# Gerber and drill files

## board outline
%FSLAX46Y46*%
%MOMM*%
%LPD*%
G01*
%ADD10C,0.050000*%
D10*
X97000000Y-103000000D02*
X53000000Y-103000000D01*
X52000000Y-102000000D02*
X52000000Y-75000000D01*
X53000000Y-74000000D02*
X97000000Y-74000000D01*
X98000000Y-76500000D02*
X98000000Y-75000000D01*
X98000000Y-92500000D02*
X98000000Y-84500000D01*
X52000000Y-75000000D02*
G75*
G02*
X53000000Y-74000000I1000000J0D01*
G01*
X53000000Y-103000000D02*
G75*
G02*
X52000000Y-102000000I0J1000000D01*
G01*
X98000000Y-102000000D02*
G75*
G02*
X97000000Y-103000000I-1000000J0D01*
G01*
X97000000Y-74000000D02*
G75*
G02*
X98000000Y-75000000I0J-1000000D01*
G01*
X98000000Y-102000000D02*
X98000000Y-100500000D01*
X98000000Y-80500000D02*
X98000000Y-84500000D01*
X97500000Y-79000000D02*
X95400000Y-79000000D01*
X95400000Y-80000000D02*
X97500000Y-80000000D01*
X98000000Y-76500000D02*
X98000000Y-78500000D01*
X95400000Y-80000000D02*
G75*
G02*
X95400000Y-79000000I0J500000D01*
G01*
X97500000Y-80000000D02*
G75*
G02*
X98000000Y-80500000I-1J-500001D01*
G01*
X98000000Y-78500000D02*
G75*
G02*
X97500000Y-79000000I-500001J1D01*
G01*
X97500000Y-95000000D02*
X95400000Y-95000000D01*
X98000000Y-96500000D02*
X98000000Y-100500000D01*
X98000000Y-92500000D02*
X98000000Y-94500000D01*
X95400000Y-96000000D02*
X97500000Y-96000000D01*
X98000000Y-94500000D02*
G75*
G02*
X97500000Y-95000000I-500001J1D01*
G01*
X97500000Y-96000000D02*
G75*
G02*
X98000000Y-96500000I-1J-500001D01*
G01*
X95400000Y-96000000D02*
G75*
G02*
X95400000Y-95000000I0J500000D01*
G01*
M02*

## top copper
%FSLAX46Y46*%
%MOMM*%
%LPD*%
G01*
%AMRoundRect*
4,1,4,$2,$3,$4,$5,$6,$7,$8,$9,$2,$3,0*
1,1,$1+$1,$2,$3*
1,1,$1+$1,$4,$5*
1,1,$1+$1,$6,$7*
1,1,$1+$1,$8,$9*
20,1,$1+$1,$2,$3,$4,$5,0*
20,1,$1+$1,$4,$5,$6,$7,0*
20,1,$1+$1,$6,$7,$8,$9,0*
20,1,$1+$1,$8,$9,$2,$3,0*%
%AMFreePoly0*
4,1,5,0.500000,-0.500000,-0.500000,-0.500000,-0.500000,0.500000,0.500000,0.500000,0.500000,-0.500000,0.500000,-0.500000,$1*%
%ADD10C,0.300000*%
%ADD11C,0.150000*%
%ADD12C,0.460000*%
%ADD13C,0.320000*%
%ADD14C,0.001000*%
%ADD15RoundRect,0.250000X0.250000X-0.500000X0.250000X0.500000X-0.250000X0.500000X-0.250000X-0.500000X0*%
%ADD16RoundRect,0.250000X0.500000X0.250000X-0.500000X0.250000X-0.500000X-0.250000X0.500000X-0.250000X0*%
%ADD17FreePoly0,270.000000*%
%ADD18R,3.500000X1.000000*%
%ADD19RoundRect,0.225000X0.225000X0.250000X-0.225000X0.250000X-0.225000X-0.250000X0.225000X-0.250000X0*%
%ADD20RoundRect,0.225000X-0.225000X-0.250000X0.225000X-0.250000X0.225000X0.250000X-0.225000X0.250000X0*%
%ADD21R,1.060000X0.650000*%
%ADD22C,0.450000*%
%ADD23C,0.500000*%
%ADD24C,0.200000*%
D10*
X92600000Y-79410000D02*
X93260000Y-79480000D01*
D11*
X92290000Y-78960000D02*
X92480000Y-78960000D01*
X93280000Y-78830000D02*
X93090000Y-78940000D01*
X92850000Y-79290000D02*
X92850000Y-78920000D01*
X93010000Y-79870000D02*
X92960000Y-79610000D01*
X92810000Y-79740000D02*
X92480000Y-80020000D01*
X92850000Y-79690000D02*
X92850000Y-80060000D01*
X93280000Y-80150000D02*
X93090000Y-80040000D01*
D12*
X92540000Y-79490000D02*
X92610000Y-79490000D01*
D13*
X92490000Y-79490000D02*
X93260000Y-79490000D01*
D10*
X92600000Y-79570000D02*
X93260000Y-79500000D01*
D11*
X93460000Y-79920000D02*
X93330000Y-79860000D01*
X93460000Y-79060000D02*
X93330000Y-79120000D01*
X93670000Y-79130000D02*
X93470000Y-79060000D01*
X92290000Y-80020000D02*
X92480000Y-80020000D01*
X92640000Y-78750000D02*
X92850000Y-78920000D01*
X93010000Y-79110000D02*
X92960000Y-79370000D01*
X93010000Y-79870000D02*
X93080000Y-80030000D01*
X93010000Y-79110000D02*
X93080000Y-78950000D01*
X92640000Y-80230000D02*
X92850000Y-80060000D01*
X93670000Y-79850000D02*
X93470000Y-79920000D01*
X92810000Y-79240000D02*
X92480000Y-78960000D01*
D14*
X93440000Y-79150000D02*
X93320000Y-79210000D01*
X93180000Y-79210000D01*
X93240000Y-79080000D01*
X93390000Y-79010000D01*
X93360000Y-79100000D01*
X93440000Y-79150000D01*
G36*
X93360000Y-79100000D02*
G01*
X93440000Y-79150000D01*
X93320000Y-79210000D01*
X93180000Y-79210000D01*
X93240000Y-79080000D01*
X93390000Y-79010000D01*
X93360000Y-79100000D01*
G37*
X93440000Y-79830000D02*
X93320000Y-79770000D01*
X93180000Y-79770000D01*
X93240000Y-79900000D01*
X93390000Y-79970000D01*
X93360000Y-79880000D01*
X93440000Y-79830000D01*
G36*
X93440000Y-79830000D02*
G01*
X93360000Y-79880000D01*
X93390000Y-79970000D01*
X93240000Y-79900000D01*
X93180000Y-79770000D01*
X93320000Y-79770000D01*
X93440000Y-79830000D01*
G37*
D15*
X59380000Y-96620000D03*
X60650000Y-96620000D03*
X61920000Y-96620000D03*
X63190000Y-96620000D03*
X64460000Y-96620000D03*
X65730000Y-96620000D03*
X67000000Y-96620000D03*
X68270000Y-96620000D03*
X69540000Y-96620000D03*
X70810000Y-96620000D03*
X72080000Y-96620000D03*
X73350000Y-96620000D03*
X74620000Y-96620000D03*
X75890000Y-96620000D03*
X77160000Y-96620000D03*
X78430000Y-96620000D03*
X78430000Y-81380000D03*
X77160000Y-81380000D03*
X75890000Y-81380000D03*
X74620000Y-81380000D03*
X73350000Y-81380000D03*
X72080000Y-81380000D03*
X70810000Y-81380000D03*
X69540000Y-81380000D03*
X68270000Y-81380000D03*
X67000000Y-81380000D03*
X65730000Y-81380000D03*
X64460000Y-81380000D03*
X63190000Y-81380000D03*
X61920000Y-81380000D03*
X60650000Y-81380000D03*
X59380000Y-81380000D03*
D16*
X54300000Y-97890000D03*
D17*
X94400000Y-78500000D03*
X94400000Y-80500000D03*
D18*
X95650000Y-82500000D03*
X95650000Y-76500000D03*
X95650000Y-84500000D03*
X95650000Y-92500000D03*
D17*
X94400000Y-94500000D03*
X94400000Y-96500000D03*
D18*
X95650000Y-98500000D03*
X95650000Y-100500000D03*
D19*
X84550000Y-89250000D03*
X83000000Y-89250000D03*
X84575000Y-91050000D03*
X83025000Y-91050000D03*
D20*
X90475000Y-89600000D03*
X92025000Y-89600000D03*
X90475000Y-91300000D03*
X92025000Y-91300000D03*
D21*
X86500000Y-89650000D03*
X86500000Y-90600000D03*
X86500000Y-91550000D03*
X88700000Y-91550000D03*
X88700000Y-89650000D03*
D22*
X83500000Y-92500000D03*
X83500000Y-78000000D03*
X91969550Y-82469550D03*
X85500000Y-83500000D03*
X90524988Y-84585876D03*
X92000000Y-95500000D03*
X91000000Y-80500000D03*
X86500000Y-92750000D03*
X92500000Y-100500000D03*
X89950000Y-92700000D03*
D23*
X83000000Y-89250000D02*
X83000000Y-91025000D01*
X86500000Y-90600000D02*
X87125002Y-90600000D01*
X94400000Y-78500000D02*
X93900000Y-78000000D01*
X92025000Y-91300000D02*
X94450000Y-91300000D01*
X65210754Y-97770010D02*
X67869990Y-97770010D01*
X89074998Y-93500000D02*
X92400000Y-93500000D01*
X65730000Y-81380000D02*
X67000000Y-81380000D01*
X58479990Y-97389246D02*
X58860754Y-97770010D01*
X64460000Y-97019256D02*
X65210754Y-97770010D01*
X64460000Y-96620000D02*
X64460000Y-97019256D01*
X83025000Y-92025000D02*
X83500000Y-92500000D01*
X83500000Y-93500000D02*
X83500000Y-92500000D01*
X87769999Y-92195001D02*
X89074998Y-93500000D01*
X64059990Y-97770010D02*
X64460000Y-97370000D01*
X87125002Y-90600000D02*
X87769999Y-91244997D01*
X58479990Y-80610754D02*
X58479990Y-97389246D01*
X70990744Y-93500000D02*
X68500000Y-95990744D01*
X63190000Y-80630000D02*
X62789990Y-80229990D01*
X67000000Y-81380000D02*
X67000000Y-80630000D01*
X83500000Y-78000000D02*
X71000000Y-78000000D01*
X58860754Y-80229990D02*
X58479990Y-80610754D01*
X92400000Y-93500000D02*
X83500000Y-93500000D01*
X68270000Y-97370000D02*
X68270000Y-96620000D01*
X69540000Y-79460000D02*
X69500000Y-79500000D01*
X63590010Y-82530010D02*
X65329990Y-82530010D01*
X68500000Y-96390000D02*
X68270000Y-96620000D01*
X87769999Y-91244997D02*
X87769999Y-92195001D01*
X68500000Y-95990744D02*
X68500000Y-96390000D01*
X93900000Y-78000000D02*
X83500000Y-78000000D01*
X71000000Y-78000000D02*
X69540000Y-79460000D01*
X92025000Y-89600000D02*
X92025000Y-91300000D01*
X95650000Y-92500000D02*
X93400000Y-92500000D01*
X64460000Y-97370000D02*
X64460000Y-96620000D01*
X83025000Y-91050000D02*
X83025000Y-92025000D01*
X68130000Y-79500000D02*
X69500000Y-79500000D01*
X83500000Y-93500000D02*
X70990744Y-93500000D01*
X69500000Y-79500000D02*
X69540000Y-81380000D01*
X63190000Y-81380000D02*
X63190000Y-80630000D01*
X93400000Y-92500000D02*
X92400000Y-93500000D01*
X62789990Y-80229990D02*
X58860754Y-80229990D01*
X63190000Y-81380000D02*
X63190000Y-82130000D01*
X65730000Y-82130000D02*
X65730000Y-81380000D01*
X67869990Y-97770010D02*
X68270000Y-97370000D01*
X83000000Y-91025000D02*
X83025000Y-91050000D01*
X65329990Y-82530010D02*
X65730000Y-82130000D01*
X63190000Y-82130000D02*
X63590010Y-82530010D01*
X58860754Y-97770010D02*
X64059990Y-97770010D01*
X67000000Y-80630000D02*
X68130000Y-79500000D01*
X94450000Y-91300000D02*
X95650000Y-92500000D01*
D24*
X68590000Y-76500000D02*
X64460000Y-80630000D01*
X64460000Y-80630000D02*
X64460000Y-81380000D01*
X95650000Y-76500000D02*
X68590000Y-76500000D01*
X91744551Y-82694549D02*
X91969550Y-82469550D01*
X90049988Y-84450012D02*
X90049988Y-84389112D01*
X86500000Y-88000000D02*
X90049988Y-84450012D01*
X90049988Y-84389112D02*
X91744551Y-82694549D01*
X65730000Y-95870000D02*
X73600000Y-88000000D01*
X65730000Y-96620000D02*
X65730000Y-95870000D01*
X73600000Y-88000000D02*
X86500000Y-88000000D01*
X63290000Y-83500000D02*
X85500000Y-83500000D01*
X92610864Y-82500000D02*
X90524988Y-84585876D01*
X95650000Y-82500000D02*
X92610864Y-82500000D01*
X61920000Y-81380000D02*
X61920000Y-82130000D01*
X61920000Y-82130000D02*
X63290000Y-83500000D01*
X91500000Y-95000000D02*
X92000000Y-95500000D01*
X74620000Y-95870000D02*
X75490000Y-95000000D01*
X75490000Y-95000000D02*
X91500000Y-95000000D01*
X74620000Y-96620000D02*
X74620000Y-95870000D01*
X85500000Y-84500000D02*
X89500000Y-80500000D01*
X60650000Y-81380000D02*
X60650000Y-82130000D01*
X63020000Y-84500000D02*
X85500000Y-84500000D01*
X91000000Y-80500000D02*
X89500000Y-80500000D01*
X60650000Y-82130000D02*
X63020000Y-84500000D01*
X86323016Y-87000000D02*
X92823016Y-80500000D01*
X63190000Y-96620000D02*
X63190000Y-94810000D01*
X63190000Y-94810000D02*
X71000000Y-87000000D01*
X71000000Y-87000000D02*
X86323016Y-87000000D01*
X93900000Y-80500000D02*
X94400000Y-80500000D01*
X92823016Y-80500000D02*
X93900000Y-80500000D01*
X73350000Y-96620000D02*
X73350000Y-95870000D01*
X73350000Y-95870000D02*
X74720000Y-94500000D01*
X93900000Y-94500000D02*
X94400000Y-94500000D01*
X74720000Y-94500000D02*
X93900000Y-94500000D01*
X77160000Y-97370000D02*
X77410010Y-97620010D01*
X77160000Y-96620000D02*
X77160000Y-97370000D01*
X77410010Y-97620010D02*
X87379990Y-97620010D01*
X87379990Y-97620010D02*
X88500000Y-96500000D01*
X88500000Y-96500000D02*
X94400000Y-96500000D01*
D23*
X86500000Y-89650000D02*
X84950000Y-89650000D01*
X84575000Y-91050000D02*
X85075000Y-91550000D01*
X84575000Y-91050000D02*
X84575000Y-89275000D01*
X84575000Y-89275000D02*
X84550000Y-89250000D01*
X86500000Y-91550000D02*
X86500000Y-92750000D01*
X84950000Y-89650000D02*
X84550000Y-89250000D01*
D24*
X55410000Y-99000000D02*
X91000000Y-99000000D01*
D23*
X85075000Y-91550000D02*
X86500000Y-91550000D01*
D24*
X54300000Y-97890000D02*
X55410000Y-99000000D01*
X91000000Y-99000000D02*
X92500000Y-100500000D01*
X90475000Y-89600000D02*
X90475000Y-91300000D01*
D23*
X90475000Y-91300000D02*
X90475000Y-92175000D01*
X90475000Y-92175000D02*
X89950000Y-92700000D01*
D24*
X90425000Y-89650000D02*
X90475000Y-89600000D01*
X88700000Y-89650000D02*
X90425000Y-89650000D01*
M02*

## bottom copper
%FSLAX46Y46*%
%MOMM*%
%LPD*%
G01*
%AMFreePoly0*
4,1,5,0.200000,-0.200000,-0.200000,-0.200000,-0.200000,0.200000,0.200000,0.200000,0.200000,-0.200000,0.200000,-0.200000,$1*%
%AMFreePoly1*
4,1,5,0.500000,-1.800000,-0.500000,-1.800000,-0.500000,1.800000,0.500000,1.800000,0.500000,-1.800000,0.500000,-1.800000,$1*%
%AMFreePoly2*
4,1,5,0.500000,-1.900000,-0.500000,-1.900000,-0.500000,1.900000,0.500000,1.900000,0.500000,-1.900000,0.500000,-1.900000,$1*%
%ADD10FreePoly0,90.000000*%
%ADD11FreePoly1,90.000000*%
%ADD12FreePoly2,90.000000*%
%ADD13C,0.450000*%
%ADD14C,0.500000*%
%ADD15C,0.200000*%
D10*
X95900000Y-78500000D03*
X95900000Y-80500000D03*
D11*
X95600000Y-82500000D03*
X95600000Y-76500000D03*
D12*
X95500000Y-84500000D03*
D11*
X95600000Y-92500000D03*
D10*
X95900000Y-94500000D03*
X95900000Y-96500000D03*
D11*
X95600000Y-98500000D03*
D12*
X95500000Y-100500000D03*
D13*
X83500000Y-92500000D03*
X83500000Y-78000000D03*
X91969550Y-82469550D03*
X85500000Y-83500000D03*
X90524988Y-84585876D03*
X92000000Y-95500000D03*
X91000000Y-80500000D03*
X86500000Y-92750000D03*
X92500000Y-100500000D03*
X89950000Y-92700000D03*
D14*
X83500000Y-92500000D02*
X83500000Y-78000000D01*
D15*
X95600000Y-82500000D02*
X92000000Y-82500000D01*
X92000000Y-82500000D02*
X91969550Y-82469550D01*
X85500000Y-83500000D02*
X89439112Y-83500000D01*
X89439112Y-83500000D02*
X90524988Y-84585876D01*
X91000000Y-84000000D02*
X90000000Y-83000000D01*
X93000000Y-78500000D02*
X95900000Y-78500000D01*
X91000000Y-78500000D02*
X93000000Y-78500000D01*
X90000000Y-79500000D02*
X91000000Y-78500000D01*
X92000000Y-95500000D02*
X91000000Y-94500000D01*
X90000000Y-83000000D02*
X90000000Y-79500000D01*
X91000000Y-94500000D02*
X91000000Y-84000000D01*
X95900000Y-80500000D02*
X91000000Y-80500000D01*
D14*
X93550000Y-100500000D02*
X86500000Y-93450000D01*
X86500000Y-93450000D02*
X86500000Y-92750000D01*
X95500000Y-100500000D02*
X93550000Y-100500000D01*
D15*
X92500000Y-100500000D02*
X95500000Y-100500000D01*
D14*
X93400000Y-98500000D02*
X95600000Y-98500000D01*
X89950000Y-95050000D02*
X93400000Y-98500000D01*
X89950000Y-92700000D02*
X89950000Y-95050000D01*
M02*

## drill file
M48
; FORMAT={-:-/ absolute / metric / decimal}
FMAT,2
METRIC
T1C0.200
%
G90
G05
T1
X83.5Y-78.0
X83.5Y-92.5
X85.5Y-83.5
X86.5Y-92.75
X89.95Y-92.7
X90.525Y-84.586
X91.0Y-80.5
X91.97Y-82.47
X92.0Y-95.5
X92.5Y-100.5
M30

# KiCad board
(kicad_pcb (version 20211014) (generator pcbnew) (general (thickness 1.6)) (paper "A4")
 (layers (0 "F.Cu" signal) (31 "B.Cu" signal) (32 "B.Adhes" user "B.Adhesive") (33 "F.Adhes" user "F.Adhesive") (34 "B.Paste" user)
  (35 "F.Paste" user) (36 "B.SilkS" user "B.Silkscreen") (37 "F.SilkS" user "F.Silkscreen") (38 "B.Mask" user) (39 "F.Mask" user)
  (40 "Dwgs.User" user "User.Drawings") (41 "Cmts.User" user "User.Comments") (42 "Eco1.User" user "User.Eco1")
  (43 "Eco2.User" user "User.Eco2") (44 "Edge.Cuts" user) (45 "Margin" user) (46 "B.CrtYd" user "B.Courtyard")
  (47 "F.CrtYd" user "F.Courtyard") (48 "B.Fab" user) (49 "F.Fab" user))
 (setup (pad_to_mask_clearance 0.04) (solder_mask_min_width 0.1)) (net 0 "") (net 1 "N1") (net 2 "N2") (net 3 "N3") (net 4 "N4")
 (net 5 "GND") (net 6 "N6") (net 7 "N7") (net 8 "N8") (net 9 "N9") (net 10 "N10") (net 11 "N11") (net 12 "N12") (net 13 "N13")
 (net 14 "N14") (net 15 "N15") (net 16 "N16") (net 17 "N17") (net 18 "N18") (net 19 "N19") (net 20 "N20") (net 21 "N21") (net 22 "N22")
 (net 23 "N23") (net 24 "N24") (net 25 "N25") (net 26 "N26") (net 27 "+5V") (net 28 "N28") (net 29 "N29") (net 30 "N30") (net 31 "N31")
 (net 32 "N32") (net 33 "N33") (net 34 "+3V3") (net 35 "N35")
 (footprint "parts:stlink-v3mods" (layer "F.Cu") (at 67 89 90)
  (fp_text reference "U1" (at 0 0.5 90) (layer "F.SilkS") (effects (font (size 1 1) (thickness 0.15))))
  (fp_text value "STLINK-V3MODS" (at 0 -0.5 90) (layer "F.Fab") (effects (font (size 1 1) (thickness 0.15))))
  (pad "1" smd roundrect locked (at -7.62 -7.62 90) (size 1.5 1) (layers "F.Cu" "F.Paste" "F.Mask") (roundrect_rratio 0.25) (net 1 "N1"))
  (pad "2" smd roundrect locked (at -7.62 -6.35 90) (size 1.5 1) (layers "F.Cu" "F.Paste" "F.Mask") (roundrect_rratio 0.25) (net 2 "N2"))
  (pad "3" smd roundrect locked (at -7.62 -5.08 90) (size 1.5 1) (layers "F.Cu" "F.Paste" "F.Mask") (roundrect_rratio 0.25) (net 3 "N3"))
  (pad "4" smd roundrect locked (at -7.62 -3.81 90) (size 1.5 1) (layers "F.Cu" "F.Paste" "F.Mask") (roundrect_rratio 0.25) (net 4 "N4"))
  (pad "5" smd roundrect locked (at -7.62 -2.54 90) (size 1.5 1) (layers "F.Cu" "F.Paste" "F.Mask") (roundrect_rratio 0.25) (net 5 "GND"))
  (pad "6" smd roundrect locked (at -7.62 -1.27 90) (size 1.5 1) (layers "F.Cu" "F.Paste" "F.Mask") (roundrect_rratio 0.25) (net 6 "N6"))
  (pad "7" smd roundrect locked (at -7.62 0 90) (size 1.5 1) (layers "F.Cu" "F.Paste" "F.Mask") (roundrect_rratio 0.25) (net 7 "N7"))
  (pad "8" smd roundrect locked (at -7.62 1.27 90) (size 1.5 1) (layers "F.Cu" "F.Paste" "F.Mask") (roundrect_rratio 0.25) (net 5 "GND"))
  (pad "9" smd roundrect locked (at -7.62 2.54 90) (size 1.5 1) (layers "F.Cu" "F.Paste" "F.Mask") (roundrect_rratio 0.25) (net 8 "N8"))
  (pad "10" smd roundrect locked (at -7.62 3.81 90) (size 1.5 1) (layers "F.Cu" "F.Paste" "F.Mask") (roundrect_rratio 0.25) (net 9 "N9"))
  (pad "11" smd roundrect locked (at -7.62 5.08 90) (size 1.5 1) (layers "F.Cu" "F.Paste" "F.Mask") (roundrect_rratio 0.25) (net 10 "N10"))
  (pad "12" smd roundrect locked (at -7.62 6.35 90) (size 1.5 1) (layers "F.Cu" "F.Paste" "F.Mask") (roundrect_rratio 0.25) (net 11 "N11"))
  (pad "13" smd roundrect locked (at -7.62 7.62 90) (size 1.5 1) (layers "F.Cu" "F.Paste" "F.Mask") (roundrect_rratio 0.25) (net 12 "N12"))
  (pad "14" smd roundrect locked (at -7.62 8.89 90) (size 1.5 1) (layers "F.Cu" "F.Paste" "F.Mask") (roundrect_rratio 0.25) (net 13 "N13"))
  (pad "15" smd roundrect locked (at -7.62 10.16 90) (size 1.5 1) (layers "F.Cu" "F.Paste" "F.Mask") (roundrect_rratio 0.25) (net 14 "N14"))
  (pad "16" smd roundrect locked (at -7.62 11.43 90) (size 1.5 1) (layers "F.Cu" "F.Paste" "F.Mask") (roundrect_rratio 0.25) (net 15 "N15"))
  (pad "17" smd roundrect locked (at 7.62 11.43 90) (size 1.5 1) (layers "F.Cu" "F.Paste" "F.Mask") (roundrect_rratio 0.25) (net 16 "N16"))
  (pad "18" smd roundrect locked (at 7.62 10.16 90) (size 1.5 1) (layers "F.Cu" "F.Paste" "F.Mask") (roundrect_rratio 0.25) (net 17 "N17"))
  (pad "19" smd roundrect locked (at 7.62 8.89 90) (size 1.5 1) (layers "F.Cu" "F.Paste" "F.Mask") (roundrect_rratio 0.25) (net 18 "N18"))
  (pad "20" smd roundrect locked (at 7.62 7.62 90) (size 1.5 1) (layers "F.Cu" "F.Paste" "F.Mask") (roundrect_rratio 0.25) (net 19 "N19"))
  (pad "21" smd roundrect locked (at 7.62 6.35 90) (size 1.5 1) (layers "F.Cu" "F.Paste" "F.Mask") (roundrect_rratio 0.25) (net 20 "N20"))
  (pad "22" smd roundrect locked (at 7.62 5.08 90) (size 1.5 1) (layers "F.Cu" "F.Paste" "F.Mask") (roundrect_rratio 0.25))
  (pad "23" smd roundrect locked (at 7.62 3.81 90) (size 1.5 1) (layers "F.Cu" "F.Paste" "F.Mask") (roundrect_rratio 0.25) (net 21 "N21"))
  (pad "24" smd roundrect locked (at 7.62 2.54 90) (size 1.5 1) (layers "F.Cu" "F.Paste" "F.Mask") (roundrect_rratio 0.25) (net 5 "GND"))
  (pad "25" smd roundrect locked (at 7.62 1.27 90) (size 1.5 1) (layers "F.Cu" "F.Paste" "F.Mask") (roundrect_rratio 0.25) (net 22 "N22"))
  (pad "26" smd roundrect locked (at 7.62 0 90) (size 1.5 1) (layers "F.Cu" "F.Paste" "F.Mask") (roundrect_rratio 0.25) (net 5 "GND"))
  (pad "27" smd roundrect locked (at 7.62 -1.27 90) (size 1.5 1) (layers "F.Cu" "F.Paste" "F.Mask") (roundrect_rratio 0.25) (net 5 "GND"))
  (pad "28" smd roundrect locked (at 7.62 -2.54 90) (size 1.5 1) (layers "F.Cu" "F.Paste" "F.Mask") (roundrect_rratio 0.25) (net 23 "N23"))
  (pad "29" smd roundrect locked (at 7.62 -3.81 90) (size 1.5 1) (layers "F.Cu" "F.Paste" "F.Mask") (roundrect_rratio 0.25) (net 5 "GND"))
  (pad "30" smd roundrect locked (at 7.62 -5.08 90) (size 1.5 1) (layers "F.Cu" "F.Paste" "F.Mask") (roundrect_rratio 0.25) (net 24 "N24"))
  (pad "31" smd roundrect locked (at 7.62 -6.35 90) (size 1.5 1) (layers "F.Cu" "F.Paste" "F.Mask") (roundrect_rratio 0.25) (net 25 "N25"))
  (pad "32" smd roundrect locked (at 7.62 -7.62 90) (size 1.5 1) (layers "F.Cu" "F.Paste" "F.Mask") (roundrect_rratio 0.25) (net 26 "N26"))
  (pad "33" smd roundrect locked (at -8.89 -12.7 180) (size 1.5 1) (layers "F.Cu" "F.Paste" "F.Mask") (roundrect_rratio 0.25) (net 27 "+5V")))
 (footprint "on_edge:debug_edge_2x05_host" (layer "F.Cu") (at 98 80.5 -90)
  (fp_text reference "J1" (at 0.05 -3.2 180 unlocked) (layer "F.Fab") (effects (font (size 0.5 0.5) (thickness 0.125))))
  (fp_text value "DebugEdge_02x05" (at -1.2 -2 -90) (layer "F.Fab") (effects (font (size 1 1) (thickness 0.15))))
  (fp_line (start -1.09 5.4) (end -1.02 4.74) (layer "F.Cu") (width 0.3))
  (fp_line (start -1.54 5.71) (end -1.54 5.52) (layer "F.Cu") (width 0.15))
  (fp_line (start -1.67 4.72) (end -1.56 4.91) (layer "F.Cu") (width 0.15))
  (fp_line (start -1.21 5.15) (end -1.58 5.15) (layer "F.Cu") (width 0.15))
  (fp_line (start -0.63 4.99) (end -0.89 5.04) (layer "F.Cu") (width 0.15))
  (fp_line (start -0.76 5.19) (end -0.48 5.52) (layer "F.Cu") (width 0.15))
  (fp_line (start -0.81 5.15) (end -0.44 5.15) (layer "F.Cu") (width 0.15))
  (fp_line (start -0.35 4.72) (end -0.46 4.91) (layer "F.Cu") (width 0.15))
  (fp_line (start -1.01 5.46) (end -1.01 5.39) (layer "F.Cu") (width 0.46))
  (fp_line (start -1.01 5.51) (end -1.01 4.74) (layer "F.Cu") (width 0.32))
  (fp_line (start -0.93 5.4) (end -1 4.74) (layer "F.Cu") (width 0.3))
  (fp_line (start -0.58 4.54) (end -0.64 4.67) (layer "F.Cu") (width 0.15))
  (fp_line (start -1.44 4.54) (end -1.38 4.67) (layer "F.Cu") (width 0.15))
  (fp_line (start -1.37 4.33) (end -1.44 4.53) (layer "F.Cu") (width 0.15))
  (fp_line (start -0.48 5.71) (end -0.48 5.52) (layer "F.Cu") (width 0.15))
  (fp_line (start -1.75 5.36) (end -1.58 5.15) (layer "F.Cu") (width 0.15))
  (fp_line (start -1.39 4.99) (end -1.13 5.04) (layer "F.Cu") (width 0.15))
  (fp_line (start -0.63 4.99) (end -0.47 4.92) (layer "F.Cu") (width 0.15))
  (fp_line (start -1.39 4.99) (end -1.55 4.92) (layer "F.Cu") (width 0.15))
  (fp_line (start -0.27 5.36) (end -0.44 5.15) (layer "F.Cu") (width 0.15))
  (fp_line (start -0.65 4.33) (end -0.58 4.53) (layer "F.Cu") (width 0.15))
  (fp_line (start -1.26 5.19) (end -1.54 5.52) (layer "F.Cu") (width 0.15))
  (fp_poly
   (pts (xy -1.35 4.56) (xy -1.29 4.68) (xy -1.29 4.82) (xy -1.42 4.76) (xy -1.49 4.61) (xy -1.4 4.64)) (layer "F.Cu") (width 0.001)
   (fill solid))
  (fp_poly
   (pts (xy -0.67 4.56) (xy -0.73 4.68) (xy -0.73 4.82) (xy -0.6 4.76) (xy -0.53 4.61) (xy -0.62 4.64)) (layer "F.Cu") (width 0.001)
   (fill solid))
  (fp_line (start 0 0) (end 4 0) (layer "Edge.Cuts") (width 0.05))
  (fp_line (start -1.5 0.5) (end -1.5 2.6) (layer "Edge.Cuts") (width 0.05))
  (fp_line (start -0.5 2.6) (end -0.5 0.5) (layer "Edge.Cuts") (width 0.05))
  (fp_line (start -4 0) (end -2 0) (layer "Edge.Cuts") (width 0.05))
  (fp_arc (start -0.5 2.6) (mid -1 3.1) (end -1.5 2.6) (layer "Edge.Cuts") (width 0.05))
  (fp_arc (start -0.5 0.5) (mid -0.353553 0.146447) (end 0 0) (layer "Edge.Cuts") (width 0.05))
  (fp_arc (start -2 0) (mid -1.646447 0.146447) (end -1.5 0.5) (layer "Edge.Cuts") (width 0.05))
  (pad "1" smd custom locked (at -2 3.6 270) (size 1 1) (layers "F.Cu" "F.Mask") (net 5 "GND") (zone_connect 0)
   (options (clearance outline) (anchor rect)) (primitives))
  (pad "2" smd custom locked (at 0 3.6 270) (size 1 1) (layers "F.Cu" "F.Mask") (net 4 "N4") (zone_connect 0)
   (options (clearance outline) (anchor rect)) (primitives))
  (pad "3" smd custom locked (at -2 2.1 90) (size 0.4 0.4) (layers "B.Cu" "B.Mask") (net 12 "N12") (zone_connect 0)
   (options (clearance outline) (anchor rect)) (primitives))
  (pad "4" smd custom locked (at 0 2.1 90) (size 0.4 0.4) (layers "B.Cu" "B.Mask") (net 25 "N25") (zone_connect 0)
   (options (clearance outline) (anchor rect)) (primitives))
  (pad "5" smd rect locked (at 2 2.35 270) (size 1 3.5) (layers "F.Cu" "F.Mask") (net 24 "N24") (zone_connect 0))
  (pad "6" smd custom locked (at 2 2.4 90) (size 1 3.6) (layers "B.Cu" "B.Mask") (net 6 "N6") (zone_connect 0)
   (options (clearance outline) (anchor rect)) (primitives))
  (pad "7" smd rect locked (at -4 2.35 270) (size 1 3.5) (layers "F.Cu" "F.Mask") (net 23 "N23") (zone_connect 0))
  (pad "8" smd custom locked (at -4 2.4 90) (size 1 3.6) (layers "B.Cu" "B.Mask") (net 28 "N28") (zone_connect 0)
   (options (clearance outline) (anchor rect)) (primitives))
  (pad "9" smd rect locked (at 4 2.35 270) (size 1 3.5) (layers "F.Cu" "F.Mask") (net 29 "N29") (zone_connect 0))
  (pad "10" smd custom locked (at 4 2.5 90) (size 1 3.8) (layers "B.Cu" "B.Mask") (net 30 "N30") (zone_connect 0)
   (options (clearance outline) (anchor rect)) (primitives)))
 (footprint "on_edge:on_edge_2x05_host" (layer "F.Cu") (at 98 96.5 -90)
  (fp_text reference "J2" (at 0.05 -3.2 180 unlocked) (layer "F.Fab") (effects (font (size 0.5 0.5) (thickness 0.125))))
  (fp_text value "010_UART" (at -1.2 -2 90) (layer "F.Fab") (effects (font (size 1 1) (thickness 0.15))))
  (fp_line (start -1.5 0.5) (end -1.5 2.6) (layer "Edge.Cuts") (width 0.05))
  (fp_line (start 0 0) (end 4 0) (layer "Edge.Cuts") (width 0.05))
  (fp_line (start -4 0) (end -2 0) (layer "Edge.Cuts") (width 0.05))
  (fp_line (start -0.5 2.6) (end -0.5 0.5) (layer "Edge.Cuts") (width 0.05))
  (fp_arc (start -2 0) (mid -1.646447 0.146447) (end -1.5 0.5) (layer "Edge.Cuts") (width 0.05))
  (fp_arc (start -0.5 0.5) (mid -0.353553 0.146447) (end 0 0) (layer "Edge.Cuts") (width 0.05))
  (fp_arc (start -0.5 2.6) (mid -1 3.1) (end -1.5 2.6) (layer "Edge.Cuts") (width 0.05))
  (pad "1" smd rect locked (at -4 2.35 270) (size 1 3.5) (layers "F.Cu" "F.Mask") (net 5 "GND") (zone_connect 0))
  (pad "2" smd custom locked (at -2 3.6 270) (size 1 1) (layers "F.Cu" "F.Mask") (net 11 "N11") (zone_connect 0)
   (options (clearance outline) (anchor rect)) (primitives))
  (pad "3" smd custom locked (at 0 3.6 270) (size 1 1) (layers "F.Cu" "F.Mask") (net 14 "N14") (zone_connect 0)
   (options (clearance outline) (anchor rect)) (primitives))
  (pad "4" smd rect locked (at 2 2.35 270) (size 1 3.5) (layers "F.Cu" "F.Mask") (zone_connect 0))
  (pad "5" smd rect locked (at 4 2.35 270) (size 1 3.5) (layers "F.Cu" "F.Mask") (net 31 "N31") (zone_connect 0))
  (pad "6" smd custom locked (at -4 2.4 90) (size 1 3.6) (layers "B.Cu" "B.Mask") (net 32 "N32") (zone_connect 0)
   (options (clearance outline) (anchor rect)) (primitives))
  (pad "7" smd custom locked (at -2 2.1 90) (size 0.4 0.4) (layers "B.Cu" "B.Mask") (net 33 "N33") (zone_connect 0)
   (options (clearance outline) (anchor rect)) (primitives))
  (pad "8" smd custom locked (at 0 2.1 90) (size 0.4 0.4) (layers "B.Cu" "B.Mask") (zone_connect 0)
   (options (clearance outline) (anchor rect)) (primitives))
  (pad "9" smd custom locked (at 2 2.4 90) (size 1 3.6) (layers "B.Cu" "B.Mask") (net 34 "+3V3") (zone_connect 0)
   (options (clearance outline) (anchor rect)) (primitives))
  (pad "10" smd custom locked (at 4 2.5 90) (size 1 3.8) (layers "B.Cu" "B.Mask") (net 27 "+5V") (zone_connect 0)
   (options (clearance outline) (anchor rect)) (primitives)))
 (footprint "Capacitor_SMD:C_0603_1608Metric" (layer "F.Cu") (at 83.775 89.25 180)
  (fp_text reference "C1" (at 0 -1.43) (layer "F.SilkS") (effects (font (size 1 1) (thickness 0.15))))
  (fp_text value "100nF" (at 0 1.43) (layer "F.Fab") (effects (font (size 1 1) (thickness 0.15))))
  (pad "1" smd roundrect locked (at -0.775 0 180) (size 0.9 0.95) (layers "F.Cu" "F.Paste" "F.Mask") (roundrect_rratio 0.25) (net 27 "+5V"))
  (pad "2" smd roundrect locked (at 0.775 0 180) (size 0.9 0.95) (layers "F.Cu" "F.Paste" "F.Mask") (roundrect_rratio 0.25) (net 5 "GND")))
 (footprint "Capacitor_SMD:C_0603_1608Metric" (layer "F.Cu") (at 83.8 91.05 180)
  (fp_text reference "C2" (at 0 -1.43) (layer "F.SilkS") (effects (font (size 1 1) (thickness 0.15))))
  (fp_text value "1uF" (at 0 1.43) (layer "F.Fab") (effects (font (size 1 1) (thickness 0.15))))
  (pad "1" smd roundrect locked (at -0.775 0 180) (size 0.9 0.95) (layers "F.Cu" "F.Paste" "F.Mask") (roundrect_rratio 0.25) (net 27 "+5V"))
  (pad "2" smd roundrect locked (at 0.775 0 180) (size 0.9 0.95) (layers "F.Cu" "F.Paste" "F.Mask") (roundrect_rratio 0.25) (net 5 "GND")))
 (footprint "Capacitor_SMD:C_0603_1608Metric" (layer "F.Cu") (at 91.25 89.6)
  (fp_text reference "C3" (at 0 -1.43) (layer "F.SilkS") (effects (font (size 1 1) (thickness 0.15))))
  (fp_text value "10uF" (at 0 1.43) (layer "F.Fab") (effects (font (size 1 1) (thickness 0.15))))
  (pad "1" smd roundrect locked (at -0.775 0) (size 0.9 0.95) (layers "F.Cu" "F.Paste" "F.Mask") (roundrect_rratio 0.25) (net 34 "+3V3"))
  (pad "2" smd roundrect locked (at 0.775 0) (size 0.9 0.95) (layers "F.Cu" "F.Paste" "F.Mask") (roundrect_rratio 0.25) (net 5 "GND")))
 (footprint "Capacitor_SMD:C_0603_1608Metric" (layer "F.Cu") (at 91.25 91.3)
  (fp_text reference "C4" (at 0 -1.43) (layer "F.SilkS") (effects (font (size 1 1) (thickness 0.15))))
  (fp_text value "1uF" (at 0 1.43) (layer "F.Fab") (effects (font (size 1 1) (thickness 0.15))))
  (pad "1" smd roundrect locked (at -0.775 0) (size 0.9 0.95) (layers "F.Cu" "F.Paste" "F.Mask") (roundrect_rratio 0.25) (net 34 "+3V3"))
  (pad "2" smd roundrect locked (at 0.775 0) (size 0.9 0.95) (layers "F.Cu" "F.Paste" "F.Mask") (roundrect_rratio 0.25) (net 5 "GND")))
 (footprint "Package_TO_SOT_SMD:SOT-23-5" (layer "F.Cu") (at 87.6 90.6)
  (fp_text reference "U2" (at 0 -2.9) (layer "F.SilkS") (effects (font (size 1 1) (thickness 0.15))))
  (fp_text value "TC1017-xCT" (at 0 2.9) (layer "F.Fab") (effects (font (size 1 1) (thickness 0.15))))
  (pad "1" smd rect locked (at -1.1 -0.95) (size 1.06 0.65) (layers "F.Cu" "F.Paste" "F.Mask") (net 27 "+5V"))
  (pad "2" smd rect locked (at -1.1 0) (size 1.06 0.65) (layers "F.Cu" "F.Paste" "F.Mask") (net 5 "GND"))
  (pad "3" smd rect locked (at -1.1 0.95) (size 1.06 0.65) (layers "F.Cu" "F.Paste" "F.Mask") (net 27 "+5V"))
  (pad "4" smd rect locked (at 1.1 0.95) (size 1.06 0.65) (layers "F.Cu" "F.Paste" "F.Mask") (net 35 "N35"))
  (pad "5" smd rect locked (at 1.1 -0.95) (size 1.06 0.65) (layers "F.Cu" "F.Paste" "F.Mask") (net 34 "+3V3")))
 (gr_line (start 97 103) (end 53 103) (layer "Edge.Cuts") (width 0.05))
 (gr_line (start 52 102) (end 52 75) (layer "Edge.Cuts") (width 0.05))
 (gr_line (start 53 74) (end 97 74) (layer "Edge.Cuts") (width 0.05))
 (gr_line (start 98 76.5) (end 98 75) (layer "Edge.Cuts") (width 0.05))
 (gr_line (start 98 92.5) (end 98 84.5) (layer "Edge.Cuts") (width 0.05))
 (gr_arc (start 52 75) (mid 52.292893 74.292893) (end 53 74) (layer "Edge.Cuts") (width 0.05))
 (gr_arc (start 53 103) (mid 52.292893 102.707107) (end 52 102) (layer "Edge.Cuts") (width 0.05))
 (gr_arc (start 98 102) (mid 97.707107 102.707107) (end 97 103) (layer "Edge.Cuts") (width 0.05))
 (gr_arc (start 97 74) (mid 97.707107 74.292893) (end 98 75) (layer "Edge.Cuts") (width 0.05))
 (gr_line (start 98 102) (end 98 100.5) (layer "Edge.Cuts") (width 0.05))
 (segment (start 83 89.25) (end 83 91.025) (width 0.5) (layer "F.Cu") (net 5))
 (segment (start 86.5 90.6) (end 87.125002 90.6) (width 0.5) (layer "F.Cu") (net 5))
 (segment (start 94.4 78.5) (end 93.9 78) (width 0.5) (layer "F.Cu") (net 5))
 (segment (start 92.025 91.3) (end 94.45 91.3) (width 0.5) (layer "F.Cu") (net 5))
 (segment (start 65.210754 97.77001) (end 67.86999 97.77001) (width 0.5) (layer "F.Cu") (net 5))
 (segment (start 89.074998 93.5) (end 92.4 93.5) (width 0.5) (layer "F.Cu") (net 5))
 (segment (start 65.73 81.38) (end 67 81.38) (width 0.5) (layer "F.Cu") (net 5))
 (segment (start 58.47999 97.389246) (end 58.860754 97.77001) (width 0.5) (layer "F.Cu") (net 5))
 (segment (start 64.46 97.019256) (end 65.210754 97.77001) (width 0.5) (layer "F.Cu") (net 5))
 (segment (start 64.46 96.62) (end 64.46 97.019256) (width 0.5) (layer "F.Cu") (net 5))
 (segment (start 83.025 92.025) (end 83.5 92.5) (width 0.5) (layer "F.Cu") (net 5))
 (segment (start 83.5 93.5) (end 83.5 92.5) (width 0.5) (layer "F.Cu") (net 5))
 (segment (start 87.769999 92.195001) (end 89.074998 93.5) (width 0.5) (layer "F.Cu") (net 5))
 (segment (start 64.05999 97.77001) (end 64.46 97.37) (width 0.5) (layer "F.Cu") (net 5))
 (segment (start 87.125002 90.6) (end 87.769999 91.244997) (width 0.5) (layer "F.Cu") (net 5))
 (segment (start 58.47999 80.610754) (end 58.47999 97.389246) (width 0.5) (layer "F.Cu") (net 5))
 (segment (start 70.990744 93.5) (end 68.5 95.990744) (width 0.5) (layer "F.Cu") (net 5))
 (segment (start 63.19 80.63) (end 62.78999 80.22999) (width 0.5) (layer "F.Cu") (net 5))
 (segment (start 67 81.38) (end 67 80.63) (width 0.5) (layer "F.Cu") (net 5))
 (segment (start 83.5 78) (end 71 78) (width 0.5) (layer "F.Cu") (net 5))
 (segment (start 58.860754 80.22999) (end 58.47999 80.610754) (width 0.5) (layer "F.Cu") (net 5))
 (segment (start 92.4 93.5) (end 83.5 93.5) (width 0.5) (layer "F.Cu") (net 5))
 (segment (start 68.27 97.37) (end 68.27 96.62) (width 0.5) (layer "F.Cu") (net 5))
 (segment (start 69.54 79.46) (end 69.5 79.5) (width 0.5) (layer "F.Cu") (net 5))
 (segment (start 63.59001 82.53001) (end 65.32999 82.53001) (width 0.5) (layer "F.Cu") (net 5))
 (segment (start 68.5 96.39) (end 68.27 96.62) (width 0.5) (layer "F.Cu") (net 5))
 (segment (start 87.769999 91.244997) (end 87.769999 92.195001) (width 0.5) (layer "F.Cu") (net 5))
 (segment (start 68.5 95.990744) (end 68.5 96.39) (width 0.5) (layer "F.Cu") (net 5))
 (segment (start 93.9 78) (end 83.5 78) (width 0.5) (layer "F.Cu") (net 5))
 (segment (start 71 78) (end 69.54 79.46) (width 0.5) (layer "F.Cu") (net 5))
 (segment (start 92.025 89.6) (end 92.025 91.3) (width 0.5) (layer "F.Cu") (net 5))
 (segment (start 95.65 92.5) (end 93.4 92.5) (width 0.5) (layer "F.Cu") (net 5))
 (segment (start 64.46 97.37) (end 64.46 96.62) (width 0.5) (layer "F.Cu") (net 5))
 (segment (start 83.025 91.05) (end 83.025 92.025) (width 0.5) (layer "F.Cu") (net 5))
 (segment (start 68.13 79.5) (end 69.5 79.5) (width 0.5) (layer "F.Cu") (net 5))
 (segment (start 83.5 93.5) (end 70.990744 93.5) (width 0.5) (layer "F.Cu") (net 5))
 (segment (start 69.5 79.5) (end 69.54 81.38) (width 0.5) (layer "F.Cu") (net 5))
 (segment (start 63.19 81.38) (end 63.19 80.63) (width 0.5) (layer "F.Cu") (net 5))
 (segment (start 93.4 92.5) (end 92.4 93.5) (width 0.5) (layer "F.Cu") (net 5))
 (segment (start 62.78999 80.22999) (end 58.860754 80.22999) (width 0.5) (layer "F.Cu") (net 5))
 (segment (start 63.19 81.38) (end 63.19 82.13) (width 0.5) (layer "F.Cu") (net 5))
 (segment (start 65.73 82.13) (end 65.73 81.38) (width 0.5) (layer "F.Cu") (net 5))
 (segment (start 67.86999 97.77001) (end 68.27 97.37) (width 0.5) (layer "F.Cu") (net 5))
 (segment (start 83 91.025) (end 83.025 91.05) (width 0.5) (layer "F.Cu") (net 5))
 (segment (start 65.32999 82.53001) (end 65.73 82.13) (width 0.5) (layer "F.Cu") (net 5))
 (segment (start 63.19 82.13) (end 63.59001 82.53001) (width 0.5) (layer "F.Cu") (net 5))
 (segment (start 58.860754 97.77001) (end 64.05999 97.77001) (width 0.5) (layer "F.Cu") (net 5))
 (segment (start 67 80.63) (end 68.13 79.5) (width 0.5) (layer "F.Cu") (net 5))
 (segment (start 94.45 91.3) (end 95.65 92.5) (width 0.5) (layer "F.Cu") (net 5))
 (via (at 83.5 92.5) (size 0.45) (drill 0.2) (layers "F.Cu" "B.Cu") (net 5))
 (via (at 83.5 78) (size 0.45) (drill 0.2) (layers "F.Cu" "B.Cu") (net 5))
 (segment (start 83.5 92.5) (end 83.5 78) (width 0.5) (layer "B.Cu") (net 5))
 (segment (start 68.59 76.5) (end 64.46 80.63) (width 0.2) (layer "F.Cu") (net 23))
 (segment (start 64.46 80.63) (end 64.46 81.38) (width 0.2) (layer "F.Cu") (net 23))
 (segment (start 95.65 76.5) (end 68.59 76.5) (width 0.2) (layer "F.Cu") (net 23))
 (segment (start 91.744551 82.694549) (end 91.96955 82.46955) (width 0.2) (layer "F.Cu") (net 6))
 (segment (start 90.049988 84.450012) (end 90.049988 84.389112) (width 0.2) (layer "F.Cu") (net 6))
 (segment (start 86.5 88) (end 90.049988 84.450012) (width 0.2) (layer "F.Cu") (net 6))
 (segment (start 90.049988 84.389112) (end 91.744551 82.694549) (width 0.2) (layer "F.Cu") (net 6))
 (segment (start 65.73 95.87) (end 73.6 88) (width 0.2) (layer "F.Cu") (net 6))
 (segment (start 65.73 96.62) (end 65.73 95.87) (width 0.2) (layer "F.Cu") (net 6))
 (segment (start 73.6 88) (end 86.5 88) (width 0.2) (layer "F.Cu") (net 6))
 (via (at 91.96955 82.46955) (size 0.45) (drill 0.2) (layers "F.Cu" "B.Cu") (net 6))
 (segment (start 95.6 82.5) (end 92 82.5) (width 0.2) (layer "B.Cu") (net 6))
 (segment (start 92 82.5) (end 91.96955 82.46955) (width 0.2) (layer "B.Cu") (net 6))
 (segment (start 63.29 83.5) (end 85.5 83.5) (width 0.2) (layer "F.Cu") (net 24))
 (segment (start 92.610864 82.5) (end 90.524988 84.585876) (width 0.2) (layer "F.Cu") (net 24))
 (segment (start 95.65 82.5) (end 92.610864 82.5) (width 0.2) (layer "F.Cu") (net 24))
 (segment (start 61.92 81.38) (end 61.92 82.13) (width 0.2) (layer "F.Cu") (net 24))
 (segment (start 61.92 82.13) (end 63.29 83.5) (width 0.2) (layer "F.Cu") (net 24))
 (via (at 85.5 83.5) (size 0.45) (drill 0.2) (layers "F.Cu" "B.Cu") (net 24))
 (via (at 90.524988 84.585876) (size 0.45) (drill 0.2) (layers "F.Cu" "B.Cu") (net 24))
 (segment (start 85.5 83.5) (end 89.439112 83.5) (width 0.2) (layer "B.Cu") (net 24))
 (segment (start 89.439112 83.5) (end 90.524988 84.585876) (width 0.2) (layer "B.Cu") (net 24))
 (segment (start 91.5 95) (end 92 95.5) (width 0.2) (layer "F.Cu") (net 12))
 (segment (start 74.62 95.87) (end 75.49 95) (width 0.2) (layer "F.Cu") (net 12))
 (segment (start 75.49 95) (end 91.5 95) (width 0.2) (layer "F.Cu") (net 12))
 (segment (start 74.62 96.62) (end 74.62 95.87) (width 0.2) (layer "F.Cu") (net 12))
 (via (at 92 95.5) (size 0.45) (drill 0.2) (layers "F.Cu" "B.Cu") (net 12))
 (segment (start 91 84) (end 90 83) (width 0.2) (layer "B.Cu") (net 12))
 (segment (start 93 78.5) (end 95.9 78.5) (width 0.2) (layer "B.Cu") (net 12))
 (segment (start 91 78.5) (end 93 78.5) (width 0.2) (layer "B.Cu") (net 12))
 (segment (start 90 79.5) (end 91 78.5) (width 0.2) (layer "B.Cu") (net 12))
 (segment (start 92 95.5) (end 91 94.5) (width 0.2) (layer "B.Cu") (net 12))
 (segment (start 90 83) (end 90 79.5) (width 0.2) (layer "B.Cu") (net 12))
 (segment (start 91 94.5) (end 91 84) (width 0.2) (layer "B.Cu") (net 12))
 (segment (start 85.5 84.5) (end 89.5 80.5) (width 0.2) (layer "F.Cu") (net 25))
 (segment (start 60.65 81.38) (end 60.65 82.13) (width 0.2) (layer "F.Cu") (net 25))
 (segment (start 63.02 84.5) (end 85.5 84.5) (width 0.2) (layer "F.Cu") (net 25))
 (segment (start 91 80.5) (end 89.5 80.5) (width 0.2) (layer "F.Cu") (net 25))
 (segment (start 60.65 82.13) (end 63.02 84.5) (width 0.2) (layer "F.Cu") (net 25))
 (via (at 91 80.5) (size 0.45) (drill 0.2) (layers "F.Cu" "B.Cu") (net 25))
 (segment (start 95.9 80.5) (end 91 80.5) (width 0.2) (layer "B.Cu") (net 25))
 (segment (start 86.323016 87) (end 92.823016 80.5) (width 0.2) (layer "F.Cu") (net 4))
 (segment (start 63.19 96.62) (end 63.19 94.81) (width 0.2) (layer "F.Cu") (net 4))
 (segment (start 63.19 94.81) (end 71 87) (width 0.2) (layer "F.Cu") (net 4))
 (segment (start 71 87) (end 86.323016 87) (width 0.2) (layer "F.Cu") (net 4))
 (segment (start 93.9 80.5) (end 94.4 80.5) (width 0.2) (layer "F.Cu") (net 4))
 (segment (start 92.823016 80.5) (end 93.9 80.5) (width 0.2) (layer "F.Cu") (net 4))
 (segment (start 73.35 96.62) (end 73.35 95.87) (width 0.2) (layer "F.Cu") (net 11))
 (segment (start 73.35 95.87) (end 74.72 94.5) (width 0.2) (layer "F.Cu") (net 11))
 (segment (start 93.9 94.5) (end 94.4 94.5) (width 0.2) (layer "F.Cu") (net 11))
 (segment (start 74.72 94.5) (end 93.9 94.5) (width 0.2) (layer "F.Cu") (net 11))
 (segment (start 77.16 97.37) (end 77.41001 97.62001) (width 0.2) (layer "F.Cu") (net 14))
 (segment (start 77.16 96.62) (end 77.16 97.37) (width 0.2) (layer "F.Cu") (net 14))
 (segment (start 77.41001 97.62001) (end 87.37999 97.62001) (width 0.2) (layer "F.Cu") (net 14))
 (segment (start 87.37999 97.62001) (end 88.5 96.5) (width 0.2) (layer "F.Cu") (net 14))
 (segment (start 88.5 96.5) (end 94.4 96.5) (width 0.2) (layer "F.Cu") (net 14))
 (segment (start 86.5 89.65) (end 84.95 89.65) (width 0.5) (layer "F.Cu") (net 27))
 (segment (start 84.575 91.05) (end 85.075 91.55) (width 0.5) (layer "F.Cu") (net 27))
 (segment (start 84.575 91.05) (end 84.575 89.275) (width 0.5) (layer "F.Cu") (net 27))
 (segment (start 84.575 89.275) (end 84.55 89.25) (width 0.5) (layer "F.Cu") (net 27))
 (segment (start 86.5 91.55) (end 86.5 92.75) (width 0.5) (layer "F.Cu") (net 27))
 (segment (start 84.95 89.65) (end 84.55 89.25) (width 0.5) (layer "F.Cu") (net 27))
 (segment (start 55.41 99) (end 91 99) (width 0.2) (layer "F.Cu") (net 27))
 (segment (start 85.075 91.55) (end 86.5 91.55) (width 0.5) (layer "F.Cu") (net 27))
 (segment (start 54.3 97.89) (end 55.41 99) (width 0.2) (layer "F.Cu") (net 27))
 (segment (start 91 99) (end 92.5 100.5) (width 0.2) (layer "F.Cu") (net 27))
 (via (at 86.5 92.75) (size 0.45) (drill 0.2) (layers "F.Cu" "B.Cu") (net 27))
 (via (at 92.5 100.5) (size 0.45) (drill 0.2) (layers "F.Cu" "B.Cu") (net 27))
 (segment (start 93.55 100.5) (end 86.5 93.45) (width 0.5) (layer "B.Cu") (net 27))
 (segment (start 86.5 93.45) (end 86.5 92.75) (width 0.5) (layer "B.Cu") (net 27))
 (segment (start 95.5 100.5) (end 93.55 100.5) (width 0.5) (layer "B.Cu") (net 27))
 (segment (start 92.5 100.5) (end 95.5 100.5) (width 0.2) (layer "B.Cu") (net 27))
 (segment (start 90.475 89.6) (end 90.475 91.3) (width 0.2) (layer "F.Cu") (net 34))
 (segment (start 90.475 91.3) (end 90.475 92.175) (width 0.5) (layer "F.Cu") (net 34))
 (segment (start 90.475 92.175) (end 89.95 92.7) (width 0.5) (layer "F.Cu") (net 34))
 (segment (start 90.425 89.65) (end 90.475 89.6) (width 0.2) (layer "F.Cu") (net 34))
 (segment (start 88.7 89.65) (end 90.425 89.65) (width 0.2) (layer "F.Cu") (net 34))
 (via (at 89.95 92.7) (size 0.45) (drill 0.2) (layers "F.Cu" "B.Cu") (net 34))
 (segment (start 93.4 98.5) (end 95.6 98.5) (width 0.5) (layer "B.Cu") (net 34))
 (segment (start 89.95 95.05) (end 93.4 98.5) (width 0.5) (layer "B.Cu") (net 34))
 (segment (start 89.95 92.7) (end 89.95 95.05) (width 0.5) (layer "B.Cu") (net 34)))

